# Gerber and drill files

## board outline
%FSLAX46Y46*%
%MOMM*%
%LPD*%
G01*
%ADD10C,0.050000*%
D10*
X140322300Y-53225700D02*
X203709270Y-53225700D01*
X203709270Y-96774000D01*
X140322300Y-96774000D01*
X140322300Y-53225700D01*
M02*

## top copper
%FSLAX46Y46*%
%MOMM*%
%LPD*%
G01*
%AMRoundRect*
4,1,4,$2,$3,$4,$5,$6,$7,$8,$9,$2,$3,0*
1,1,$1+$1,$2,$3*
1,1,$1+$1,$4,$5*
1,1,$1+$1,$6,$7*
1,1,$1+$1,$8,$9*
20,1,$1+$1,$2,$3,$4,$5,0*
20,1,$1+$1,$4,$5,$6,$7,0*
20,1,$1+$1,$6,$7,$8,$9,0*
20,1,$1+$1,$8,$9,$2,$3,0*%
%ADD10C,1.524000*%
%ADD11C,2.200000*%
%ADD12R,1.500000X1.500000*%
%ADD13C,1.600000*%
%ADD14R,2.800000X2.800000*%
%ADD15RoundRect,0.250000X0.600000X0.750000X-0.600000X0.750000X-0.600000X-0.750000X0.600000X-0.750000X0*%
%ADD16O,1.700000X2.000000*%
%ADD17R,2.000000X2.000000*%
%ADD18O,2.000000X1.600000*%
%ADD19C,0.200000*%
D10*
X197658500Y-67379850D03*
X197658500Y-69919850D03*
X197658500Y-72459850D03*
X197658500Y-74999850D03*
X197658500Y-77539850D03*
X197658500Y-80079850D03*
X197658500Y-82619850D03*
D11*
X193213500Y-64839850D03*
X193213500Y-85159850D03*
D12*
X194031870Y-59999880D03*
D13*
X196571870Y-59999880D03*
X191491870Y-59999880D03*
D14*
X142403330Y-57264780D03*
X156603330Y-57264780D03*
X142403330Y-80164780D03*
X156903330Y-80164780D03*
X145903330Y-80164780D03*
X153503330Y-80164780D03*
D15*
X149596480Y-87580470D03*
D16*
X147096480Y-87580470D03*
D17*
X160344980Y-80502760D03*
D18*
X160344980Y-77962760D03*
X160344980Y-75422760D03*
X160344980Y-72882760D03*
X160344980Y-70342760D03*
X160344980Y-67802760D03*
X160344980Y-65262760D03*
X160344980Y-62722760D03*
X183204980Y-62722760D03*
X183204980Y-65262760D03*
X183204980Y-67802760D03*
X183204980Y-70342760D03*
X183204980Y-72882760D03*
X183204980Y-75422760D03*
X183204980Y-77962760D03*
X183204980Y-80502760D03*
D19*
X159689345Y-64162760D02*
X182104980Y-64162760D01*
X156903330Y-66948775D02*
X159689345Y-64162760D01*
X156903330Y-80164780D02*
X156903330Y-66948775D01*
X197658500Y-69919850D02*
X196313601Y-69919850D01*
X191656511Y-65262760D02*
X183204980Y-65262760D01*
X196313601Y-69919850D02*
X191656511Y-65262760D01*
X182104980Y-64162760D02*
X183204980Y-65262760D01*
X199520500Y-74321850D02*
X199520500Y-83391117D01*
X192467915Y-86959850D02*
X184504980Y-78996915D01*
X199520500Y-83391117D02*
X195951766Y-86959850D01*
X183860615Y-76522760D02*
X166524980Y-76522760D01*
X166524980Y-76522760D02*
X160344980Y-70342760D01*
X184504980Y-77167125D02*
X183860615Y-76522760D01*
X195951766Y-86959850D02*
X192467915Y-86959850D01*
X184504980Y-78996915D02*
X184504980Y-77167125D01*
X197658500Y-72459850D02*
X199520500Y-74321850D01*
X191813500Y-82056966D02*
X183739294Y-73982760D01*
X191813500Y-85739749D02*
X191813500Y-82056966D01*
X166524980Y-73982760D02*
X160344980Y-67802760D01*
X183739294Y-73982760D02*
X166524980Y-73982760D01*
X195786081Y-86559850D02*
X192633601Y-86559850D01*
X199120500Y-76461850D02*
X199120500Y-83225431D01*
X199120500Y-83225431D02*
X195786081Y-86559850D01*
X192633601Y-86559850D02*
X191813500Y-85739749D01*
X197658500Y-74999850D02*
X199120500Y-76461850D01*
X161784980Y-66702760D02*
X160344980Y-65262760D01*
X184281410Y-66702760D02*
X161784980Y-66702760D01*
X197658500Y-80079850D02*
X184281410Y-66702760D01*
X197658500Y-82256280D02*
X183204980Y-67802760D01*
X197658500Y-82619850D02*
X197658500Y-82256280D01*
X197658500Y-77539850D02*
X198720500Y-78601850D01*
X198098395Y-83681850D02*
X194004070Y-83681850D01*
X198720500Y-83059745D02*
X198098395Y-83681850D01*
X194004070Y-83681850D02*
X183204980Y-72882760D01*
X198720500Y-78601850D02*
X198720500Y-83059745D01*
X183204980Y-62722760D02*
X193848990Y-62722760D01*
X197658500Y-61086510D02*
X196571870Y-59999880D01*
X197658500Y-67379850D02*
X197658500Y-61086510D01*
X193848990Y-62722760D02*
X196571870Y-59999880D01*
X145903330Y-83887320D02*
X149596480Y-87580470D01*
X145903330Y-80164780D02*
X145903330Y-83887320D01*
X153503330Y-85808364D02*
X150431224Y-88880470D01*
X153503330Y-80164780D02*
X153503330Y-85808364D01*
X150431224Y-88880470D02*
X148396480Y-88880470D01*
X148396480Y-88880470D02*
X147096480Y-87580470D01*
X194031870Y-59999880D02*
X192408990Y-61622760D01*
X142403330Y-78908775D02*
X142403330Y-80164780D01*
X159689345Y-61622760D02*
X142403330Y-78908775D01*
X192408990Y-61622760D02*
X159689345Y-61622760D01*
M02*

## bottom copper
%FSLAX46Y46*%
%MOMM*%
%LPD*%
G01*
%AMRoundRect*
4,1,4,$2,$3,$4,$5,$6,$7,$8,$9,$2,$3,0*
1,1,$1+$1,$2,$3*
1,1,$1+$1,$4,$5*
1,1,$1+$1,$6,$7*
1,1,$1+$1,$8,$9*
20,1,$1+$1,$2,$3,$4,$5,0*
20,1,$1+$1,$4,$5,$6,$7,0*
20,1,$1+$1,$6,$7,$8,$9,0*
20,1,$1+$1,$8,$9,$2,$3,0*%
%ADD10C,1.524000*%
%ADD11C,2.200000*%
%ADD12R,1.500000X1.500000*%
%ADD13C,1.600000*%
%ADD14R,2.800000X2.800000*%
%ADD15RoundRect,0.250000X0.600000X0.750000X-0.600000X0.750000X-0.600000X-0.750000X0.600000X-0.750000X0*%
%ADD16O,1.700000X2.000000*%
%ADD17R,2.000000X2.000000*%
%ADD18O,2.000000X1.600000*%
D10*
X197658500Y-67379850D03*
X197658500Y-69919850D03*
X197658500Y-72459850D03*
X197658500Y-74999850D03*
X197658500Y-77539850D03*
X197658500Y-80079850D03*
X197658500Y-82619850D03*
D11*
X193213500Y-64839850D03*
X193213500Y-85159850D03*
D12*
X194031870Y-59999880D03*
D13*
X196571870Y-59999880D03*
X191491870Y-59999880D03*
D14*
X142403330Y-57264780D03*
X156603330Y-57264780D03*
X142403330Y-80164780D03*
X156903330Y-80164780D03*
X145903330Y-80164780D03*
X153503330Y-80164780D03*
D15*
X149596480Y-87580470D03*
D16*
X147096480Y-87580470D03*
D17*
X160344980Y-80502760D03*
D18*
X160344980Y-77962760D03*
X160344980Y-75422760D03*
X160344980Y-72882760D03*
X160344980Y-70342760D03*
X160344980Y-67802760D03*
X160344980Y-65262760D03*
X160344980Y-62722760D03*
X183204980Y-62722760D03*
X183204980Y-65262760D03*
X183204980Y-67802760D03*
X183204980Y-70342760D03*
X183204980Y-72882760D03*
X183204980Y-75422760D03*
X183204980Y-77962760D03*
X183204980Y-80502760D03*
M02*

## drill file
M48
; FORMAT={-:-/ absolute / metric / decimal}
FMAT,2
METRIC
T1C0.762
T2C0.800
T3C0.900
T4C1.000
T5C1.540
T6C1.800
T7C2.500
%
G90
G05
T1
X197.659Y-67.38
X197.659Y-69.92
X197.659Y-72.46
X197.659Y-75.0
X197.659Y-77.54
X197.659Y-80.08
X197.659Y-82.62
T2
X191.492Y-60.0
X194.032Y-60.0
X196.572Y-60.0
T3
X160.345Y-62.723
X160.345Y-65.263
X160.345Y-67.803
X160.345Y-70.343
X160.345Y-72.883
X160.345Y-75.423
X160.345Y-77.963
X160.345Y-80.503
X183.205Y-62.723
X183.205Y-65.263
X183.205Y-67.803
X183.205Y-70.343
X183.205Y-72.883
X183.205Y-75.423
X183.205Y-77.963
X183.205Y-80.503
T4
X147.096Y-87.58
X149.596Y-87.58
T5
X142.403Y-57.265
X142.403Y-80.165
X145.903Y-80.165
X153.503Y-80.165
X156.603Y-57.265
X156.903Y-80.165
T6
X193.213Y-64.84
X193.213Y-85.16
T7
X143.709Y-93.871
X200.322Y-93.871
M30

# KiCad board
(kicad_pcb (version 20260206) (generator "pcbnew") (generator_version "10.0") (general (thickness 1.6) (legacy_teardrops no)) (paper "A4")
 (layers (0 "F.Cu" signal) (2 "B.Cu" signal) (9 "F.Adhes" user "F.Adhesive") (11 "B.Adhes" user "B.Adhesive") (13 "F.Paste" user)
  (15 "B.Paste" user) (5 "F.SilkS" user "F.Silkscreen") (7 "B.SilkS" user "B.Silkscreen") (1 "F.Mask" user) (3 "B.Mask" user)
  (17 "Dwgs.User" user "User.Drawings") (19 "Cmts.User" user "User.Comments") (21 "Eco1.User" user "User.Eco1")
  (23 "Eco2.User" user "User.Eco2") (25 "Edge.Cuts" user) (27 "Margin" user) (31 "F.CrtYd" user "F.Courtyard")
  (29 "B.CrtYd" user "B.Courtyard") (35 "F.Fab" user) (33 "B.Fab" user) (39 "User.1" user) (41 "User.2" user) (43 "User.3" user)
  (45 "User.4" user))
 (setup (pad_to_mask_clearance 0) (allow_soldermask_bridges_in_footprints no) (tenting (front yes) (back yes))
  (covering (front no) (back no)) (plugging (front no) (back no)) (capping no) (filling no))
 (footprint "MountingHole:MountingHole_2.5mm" (layer "F.Cu") (at 143.70939 93.87078)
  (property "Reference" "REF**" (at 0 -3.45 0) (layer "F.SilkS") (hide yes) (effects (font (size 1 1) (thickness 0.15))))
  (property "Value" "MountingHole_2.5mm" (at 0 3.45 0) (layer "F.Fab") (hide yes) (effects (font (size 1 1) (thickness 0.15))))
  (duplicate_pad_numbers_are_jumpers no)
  (pad "" np_thru_hole circle (at 0 0) (size 2.5 2.5) (drill 2.5) (layers "*.Cu" "*.Mask")))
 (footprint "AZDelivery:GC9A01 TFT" (layer "F.Cu") (at 197.6585 67.37985)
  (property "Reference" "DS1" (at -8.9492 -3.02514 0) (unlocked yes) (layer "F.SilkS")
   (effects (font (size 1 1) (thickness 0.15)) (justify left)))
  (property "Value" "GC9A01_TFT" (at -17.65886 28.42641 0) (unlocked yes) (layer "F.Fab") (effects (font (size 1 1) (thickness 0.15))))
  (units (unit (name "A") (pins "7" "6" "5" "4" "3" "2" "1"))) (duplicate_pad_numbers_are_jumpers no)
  (pad "1" thru_hole circle (at 0 0) (size 1.524 1.524) (drill 0.762) (layers "*.Cu" "*.Mask") (remove_unused_layers no)
   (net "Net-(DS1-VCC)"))
  (pad "2" thru_hole circle (at 0 2.54) (size 1.524 1.524) (drill 0.762) (layers "*.Cu" "*.Mask") (remove_unused_layers no)
   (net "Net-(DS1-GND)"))
  (pad "3" thru_hole circle (at 0 5.08) (size 1.524 1.524) (drill 0.762) (layers "*.Cu" "*.Mask") (remove_unused_layers no)
   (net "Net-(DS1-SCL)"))
  (pad "4" thru_hole circle (at 0 7.62) (size 1.524 1.524) (drill 0.762) (layers "*.Cu" "*.Mask") (remove_unused_layers no)
   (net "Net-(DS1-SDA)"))
  (pad "5" thru_hole circle (at 0 10.16) (size 1.524 1.524) (drill 0.762) (layers "*.Cu" "*.Mask") (remove_unused_layers no)
   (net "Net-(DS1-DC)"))
  (pad "6" thru_hole circle (at 0 12.7) (size 1.524 1.524) (drill 0.762) (layers "*.Cu" "*.Mask") (remove_unused_layers no)
   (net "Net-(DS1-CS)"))
  (pad "7" thru_hole circle (at 0 15.24) (size 1.524 1.524) (drill 0.762) (layers "*.Cu" "*.Mask") (remove_unused_layers no)
   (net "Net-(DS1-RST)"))
  (pad "NC0" thru_hole circle (at -4.445 -2.54) (size 2.2 2.2) (drill 1.8) (layers "*.Cu" "*.Mask") (remove_unused_layers no))
  (pad "NC1" thru_hole circle (at -4.445 17.78) (size 2.2 2.2) (drill 1.8) (layers "*.Cu" "*.Mask") (remove_unused_layers no)))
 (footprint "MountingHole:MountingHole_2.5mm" (layer "F.Cu") (at 200.32218 93.87078)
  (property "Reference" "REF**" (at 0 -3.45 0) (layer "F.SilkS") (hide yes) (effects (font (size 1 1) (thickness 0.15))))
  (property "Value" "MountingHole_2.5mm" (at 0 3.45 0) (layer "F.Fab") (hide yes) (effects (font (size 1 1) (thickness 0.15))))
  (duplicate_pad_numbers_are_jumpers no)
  (pad "" np_thru_hole circle (at 0 0) (size 2.5 2.5) (drill 2.5) (layers "*.Cu" "*.Mask")))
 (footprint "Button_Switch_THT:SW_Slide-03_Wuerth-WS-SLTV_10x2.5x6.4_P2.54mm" (layer "F.Cu") (at 194.03187 59.99988 180)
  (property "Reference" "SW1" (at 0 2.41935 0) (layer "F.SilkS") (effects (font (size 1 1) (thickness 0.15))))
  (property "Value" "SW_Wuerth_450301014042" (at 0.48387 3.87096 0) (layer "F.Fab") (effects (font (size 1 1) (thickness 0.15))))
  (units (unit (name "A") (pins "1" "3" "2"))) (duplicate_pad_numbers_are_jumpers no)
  (pad "1" thru_hole rect (at 0 0 180) (size 1.5 1.5) (drill 0.8) (layers "*.Cu" "*.Mask") (remove_unused_layers no) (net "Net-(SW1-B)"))
  (pad "2" thru_hole circle (at -2.54 0 180) (size 1.6 1.6) (drill 0.8) (layers "*.Cu" "*.Mask") (remove_unused_layers no)
   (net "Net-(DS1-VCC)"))
  (pad "3" thru_hole circle (at 2.54 0 180) (size 1.6 1.6) (drill 0.8) (layers "*.Cu" "*.Mask") (remove_unused_layers no)
   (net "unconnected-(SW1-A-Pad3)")))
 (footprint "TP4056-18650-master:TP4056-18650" (layer "B.Cu") (at 140.70333 55.56478 -90)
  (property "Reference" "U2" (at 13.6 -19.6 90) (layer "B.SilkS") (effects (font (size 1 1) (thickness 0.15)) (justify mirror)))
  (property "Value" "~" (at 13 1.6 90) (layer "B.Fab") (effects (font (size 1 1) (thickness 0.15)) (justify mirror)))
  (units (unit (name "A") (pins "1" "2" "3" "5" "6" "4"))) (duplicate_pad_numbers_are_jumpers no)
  (pad "1" thru_hole rect (at 1.7 -1.7 270) (size 2.8 2.8) (drill 1.54) (layers "*.Cu" "*.Mask") (remove_unused_layers no)
   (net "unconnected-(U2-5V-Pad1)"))
  (pad "2" thru_hole rect (at 1.7 -15.9 270) (size 2.8 2.8) (drill 1.54) (layers "*.Cu" "*.Mask") (remove_unused_layers no)
   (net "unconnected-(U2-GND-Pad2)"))
  (pad "3" thru_hole rect (at 24.6 -1.7 270) (size 2.8 2.8) (drill 1.54) (layers "*.Cu" "*.Mask") (remove_unused_layers no)
   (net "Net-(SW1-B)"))
  (pad "4" thru_hole rect (at 24.6 -16.2 270) (size 2.8 2.8) (drill 1.54) (layers "*.Cu" "*.Mask") (remove_unused_layers no)
   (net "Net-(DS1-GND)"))
  (pad "5" thru_hole rect (at 24.6 -5.2 270) (size 2.8 2.8) (drill 1.54) (layers "*.Cu" "*.Mask") (remove_unused_layers no)
   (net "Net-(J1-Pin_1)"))
  (pad "6" thru_hole rect (at 24.6 -12.8 270) (size 2.8 2.8) (drill 1.54) (layers "*.Cu" "*.Mask") (remove_unused_layers no)
   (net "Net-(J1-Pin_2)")))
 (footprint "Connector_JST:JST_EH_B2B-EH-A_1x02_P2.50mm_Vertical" (layer "B.Cu") (at 149.59648 87.58047 180)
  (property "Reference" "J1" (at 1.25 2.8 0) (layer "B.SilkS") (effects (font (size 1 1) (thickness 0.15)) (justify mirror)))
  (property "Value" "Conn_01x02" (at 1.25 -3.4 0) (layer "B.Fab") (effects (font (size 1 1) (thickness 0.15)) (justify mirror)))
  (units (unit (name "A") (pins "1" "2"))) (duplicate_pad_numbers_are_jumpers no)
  (pad "1" thru_hole roundrect (at 0 0 180) (size 1.7 2) (drill 1) (layers "*.Cu" "*.Mask") (remove_unused_layers no)
   (roundrect_rratio 0.147059) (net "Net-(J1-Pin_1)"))
  (pad "2" thru_hole oval (at 2.5 0 180) (size 1.7 2) (drill 1) (layers "*.Cu" "*.Mask") (remove_unused_layers no) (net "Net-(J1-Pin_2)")))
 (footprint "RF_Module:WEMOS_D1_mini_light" (layer "B.Cu") (at 160.34498 80.50276)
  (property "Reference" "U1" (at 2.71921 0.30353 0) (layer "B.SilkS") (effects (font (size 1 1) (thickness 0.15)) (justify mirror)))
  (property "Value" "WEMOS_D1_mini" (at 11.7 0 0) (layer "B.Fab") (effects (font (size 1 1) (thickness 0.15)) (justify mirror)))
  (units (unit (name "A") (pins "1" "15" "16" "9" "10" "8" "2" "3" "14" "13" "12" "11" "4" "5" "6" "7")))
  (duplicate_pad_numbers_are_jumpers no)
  (pad "1" thru_hole rect (at 0 0) (size 2 2) (drill 0.9) (layers "*.Cu" "*.Mask") (remove_unused_layers no)
   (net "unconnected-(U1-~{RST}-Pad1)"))
  (pad "2" thru_hole oval (at 0 -2.54) (size 2 1.6) (drill 0.9) (layers "*.Cu" "*.Mask") (remove_unused_layers no)
   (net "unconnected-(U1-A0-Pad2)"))
  (pad "3" thru_hole oval (at 0 -5.08) (size 2 1.6) (drill 0.9) (layers "*.Cu" "*.Mask") (remove_unused_layers no)
   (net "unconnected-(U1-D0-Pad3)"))
  (pad "4" thru_hole oval (at 0 -7.62) (size 2 1.6) (drill 0.9) (layers "*.Cu" "*.Mask") (remove_unused_layers no)
   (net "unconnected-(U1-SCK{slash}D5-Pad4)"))
  (pad "5" thru_hole oval (at 0 -10.16) (size 2 1.6) (drill 0.9) (layers "*.Cu" "*.Mask") (remove_unused_layers no) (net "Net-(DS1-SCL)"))
  (pad "6" thru_hole oval (at 0 -12.7) (size 2 1.6) (drill 0.9) (layers "*.Cu" "*.Mask") (remove_unused_layers no) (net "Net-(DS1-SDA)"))
  (pad "7" thru_hole oval (at 0 -15.24) (size 2 1.6) (drill 0.9) (layers "*.Cu" "*.Mask") (remove_unused_layers no) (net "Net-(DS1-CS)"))
  (pad "8" thru_hole oval (at 0 -17.78) (size 2 1.6) (drill 0.9) (layers "*.Cu" "*.Mask") (remove_unused_layers no)
   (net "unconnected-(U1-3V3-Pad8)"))
  (pad "9" thru_hole oval (at 22.86 -17.78) (size 2 1.6) (drill 0.9) (layers "*.Cu" "*.Mask") (remove_unused_layers no)
   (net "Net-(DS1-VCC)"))
  (pad "10" thru_hole oval (at 22.86 -15.24) (size 2 1.6) (drill 0.9) (layers "*.Cu" "*.Mask") (remove_unused_layers no)
   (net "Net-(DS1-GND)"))
  (pad "11" thru_hole oval (at 22.86 -12.7) (size 2 1.6) (drill 0.9) (layers "*.Cu" "*.Mask") (remove_unused_layers no)
   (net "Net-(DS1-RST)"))
  (pad "12" thru_hole oval (at 22.86 -10.16) (size 2 1.6) (drill 0.9) (layers "*.Cu" "*.Mask") (remove_unused_layers no)
   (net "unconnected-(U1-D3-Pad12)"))
  (pad "13" thru_hole oval (at 22.86 -7.62) (size 2 1.6) (drill 0.9) (layers "*.Cu" "*.Mask") (remove_unused_layers no) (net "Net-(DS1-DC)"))
  (pad "14" thru_hole oval (at 22.86 -5.08) (size 2 1.6) (drill 0.9) (layers "*.Cu" "*.Mask") (remove_unused_layers no)
   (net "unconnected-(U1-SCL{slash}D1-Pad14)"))
  (pad "15" thru_hole oval (at 22.86 -2.54) (size 2 1.6) (drill 0.9) (layers "*.Cu" "*.Mask") (remove_unused_layers no)
   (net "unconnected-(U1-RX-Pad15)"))
  (pad "16" thru_hole oval (at 22.86 0) (size 2 1.6) (drill 0.9) (layers "*.Cu" "*.Mask") (remove_unused_layers no)
   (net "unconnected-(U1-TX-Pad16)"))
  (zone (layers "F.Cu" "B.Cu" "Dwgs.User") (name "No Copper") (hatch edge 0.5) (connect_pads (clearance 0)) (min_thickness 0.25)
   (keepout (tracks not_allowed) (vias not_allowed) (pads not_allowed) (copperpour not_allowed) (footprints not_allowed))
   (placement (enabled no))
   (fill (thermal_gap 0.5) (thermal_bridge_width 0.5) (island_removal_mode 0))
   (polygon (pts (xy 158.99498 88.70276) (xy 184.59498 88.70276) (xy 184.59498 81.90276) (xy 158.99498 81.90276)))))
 (gr_rect (start 140.3223 53.2257) (end 203.70927 96.774) (stroke (width 0.05) (type default)) (fill no) (layer "Edge.Cuts"))
 (segment (start 159.689345 64.16276) (end 182.10498 64.16276) (width 0.2) (layer "F.Cu") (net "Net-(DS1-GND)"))
 (segment (start 156.90333 66.948775) (end 159.689345 64.16276) (width 0.2) (layer "F.Cu") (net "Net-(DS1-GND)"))
 (segment (start 156.90333 80.16478) (end 156.90333 66.948775) (width 0.2) (layer "F.Cu") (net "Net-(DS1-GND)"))
 (segment (start 197.6585 69.91985) (end 196.313601 69.91985) (width 0.2) (layer "F.Cu") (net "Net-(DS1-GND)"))
 (segment (start 191.656511 65.26276) (end 183.20498 65.26276) (width 0.2) (layer "F.Cu") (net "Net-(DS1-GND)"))
 (segment (start 196.313601 69.91985) (end 191.656511 65.26276) (width 0.2) (layer "F.Cu") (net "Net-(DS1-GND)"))
 (segment (start 182.10498 64.16276) (end 183.20498 65.26276) (width 0.2) (layer "F.Cu") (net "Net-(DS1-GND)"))
 (segment (start 199.5205 74.32185) (end 199.5205 83.391117) (width 0.2) (layer "F.Cu") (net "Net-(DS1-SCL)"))
 (segment (start 192.467915 86.95985) (end 184.50498 78.996915) (width 0.2) (layer "F.Cu") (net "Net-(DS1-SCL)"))
 (segment (start 199.5205 83.391117) (end 195.951766 86.95985) (width 0.2) (layer "F.Cu") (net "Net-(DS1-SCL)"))
 (segment (start 183.860615 76.52276) (end 166.52498 76.52276) (width 0.2) (layer "F.Cu") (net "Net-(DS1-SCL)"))
 (segment (start 166.52498 76.52276) (end 160.34498 70.34276) (width 0.2) (layer "F.Cu") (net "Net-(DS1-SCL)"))
 (segment (start 184.50498 77.167125) (end 183.860615 76.52276) (width 0.2) (layer "F.Cu") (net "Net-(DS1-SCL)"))
 (segment (start 195.951766 86.95985) (end 192.467915 86.95985) (width 0.2) (layer "F.Cu") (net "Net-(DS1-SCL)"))
 (segment (start 184.50498 78.996915) (end 184.50498 77.167125) (width 0.2) (layer "F.Cu") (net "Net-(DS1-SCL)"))
 (segment (start 197.6585 72.45985) (end 199.5205 74.32185) (width 0.2) (layer "F.Cu") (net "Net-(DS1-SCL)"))
 (segment (start 191.8135 82.056966) (end 183.739294 73.98276) (width 0.2) (layer "F.Cu") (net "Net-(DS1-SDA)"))
 (segment (start 191.8135 85.739749) (end 191.8135 82.056966) (width 0.2) (layer "F.Cu") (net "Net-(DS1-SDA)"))
 (segment (start 166.52498 73.98276) (end 160.34498 67.80276) (width 0.2) (layer "F.Cu") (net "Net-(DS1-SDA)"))
 (segment (start 183.739294 73.98276) (end 166.52498 73.98276) (width 0.2) (layer "F.Cu") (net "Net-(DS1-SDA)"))
 (segment (start 195.786081 86.55985) (end 192.633601 86.55985) (width 0.2) (layer "F.Cu") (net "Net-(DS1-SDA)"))
 (segment (start 199.1205 76.46185) (end 199.1205 83.225431) (width 0.2) (layer "F.Cu") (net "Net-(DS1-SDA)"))
 (segment (start 199.1205 83.225431) (end 195.786081 86.55985) (width 0.2) (layer "F.Cu") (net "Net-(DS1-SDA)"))
 (segment (start 192.633601 86.55985) (end 191.8135 85.739749) (width 0.2) (layer "F.Cu") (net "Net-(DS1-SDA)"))
 (segment (start 197.6585 74.99985) (end 199.1205 76.46185) (width 0.2) (layer "F.Cu") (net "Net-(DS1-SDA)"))
 (segment (start 161.78498 66.70276) (end 160.34498 65.26276) (width 0.2) (layer "F.Cu") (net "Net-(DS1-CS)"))
 (segment (start 184.28141 66.70276) (end 161.78498 66.70276) (width 0.2) (layer "F.Cu") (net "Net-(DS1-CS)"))
 (segment (start 197.6585 80.07985) (end 184.28141 66.70276) (width 0.2) (layer "F.Cu") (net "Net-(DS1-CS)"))
 (segment (start 197.6585 82.25628) (end 183.20498 67.80276) (width 0.2) (layer "F.Cu") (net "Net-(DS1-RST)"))
 (segment (start 197.6585 82.61985) (end 197.6585 82.25628) (width 0.2) (layer "F.Cu") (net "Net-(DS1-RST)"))
 (segment (start 197.6585 77.53985) (end 198.7205 78.60185) (width 0.2) (layer "F.Cu") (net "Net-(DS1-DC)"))
 (segment (start 198.098395 83.68185) (end 194.00407 83.68185) (width 0.2) (layer "F.Cu") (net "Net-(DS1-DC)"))
 (segment (start 198.7205 83.059745) (end 198.098395 83.68185) (width 0.2) (layer "F.Cu") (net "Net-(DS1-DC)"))
 (segment (start 194.00407 83.68185) (end 183.20498 72.88276) (width 0.2) (layer "F.Cu") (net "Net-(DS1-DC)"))
 (segment (start 198.7205 78.60185) (end 198.7205 83.059745) (width 0.2) (layer "F.Cu") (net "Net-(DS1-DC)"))
 (segment (start 183.20498 62.72276) (end 193.84899 62.72276) (width 0.2) (layer "F.Cu") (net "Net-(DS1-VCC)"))
 (segment (start 197.6585 61.08651) (end 196.57187 59.99988) (width 0.2) (layer "F.Cu") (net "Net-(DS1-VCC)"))
 (segment (start 197.6585 67.37985) (end 197.6585 61.08651) (width 0.2) (layer "F.Cu") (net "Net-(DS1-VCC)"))
 (segment (start 193.84899 62.72276) (end 196.57187 59.99988) (width 0.2) (layer "F.Cu") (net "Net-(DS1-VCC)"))
 (segment (start 145.90333 83.88732) (end 149.59648 87.58047) (width 0.2) (layer "F.Cu") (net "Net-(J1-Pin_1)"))
 (segment (start 145.90333 80.16478) (end 145.90333 83.88732) (width 0.2) (layer "F.Cu") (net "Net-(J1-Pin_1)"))
 (segment (start 153.50333 85.808364) (end 150.431224 88.88047) (width 0.2) (layer "F.Cu") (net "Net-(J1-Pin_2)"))
 (segment (start 153.50333 80.16478) (end 153.50333 85.808364) (width 0.2) (layer "F.Cu") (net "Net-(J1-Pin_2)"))
 (segment (start 150.431224 88.88047) (end 148.39648 88.88047) (width 0.2) (layer "F.Cu") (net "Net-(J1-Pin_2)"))
 (segment (start 148.39648 88.88047) (end 147.09648 87.58047) (width 0.2) (layer "F.Cu") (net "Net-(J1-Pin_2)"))
 (segment (start 194.03187 59.99988) (end 192.40899 61.62276) (width 0.2) (layer "F.Cu") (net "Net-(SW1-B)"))
 (segment (start 142.40333 78.908775) (end 142.40333 80.16478) (width 0.2) (layer "F.Cu") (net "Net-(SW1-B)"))
 (segment (start 159.689345 61.62276) (end 142.40333 78.908775) (width 0.2) (layer "F.Cu") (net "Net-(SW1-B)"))
 (segment (start 192.40899 61.62276) (end 159.689345 61.62276) (width 0.2) (layer "F.Cu") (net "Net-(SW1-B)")))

